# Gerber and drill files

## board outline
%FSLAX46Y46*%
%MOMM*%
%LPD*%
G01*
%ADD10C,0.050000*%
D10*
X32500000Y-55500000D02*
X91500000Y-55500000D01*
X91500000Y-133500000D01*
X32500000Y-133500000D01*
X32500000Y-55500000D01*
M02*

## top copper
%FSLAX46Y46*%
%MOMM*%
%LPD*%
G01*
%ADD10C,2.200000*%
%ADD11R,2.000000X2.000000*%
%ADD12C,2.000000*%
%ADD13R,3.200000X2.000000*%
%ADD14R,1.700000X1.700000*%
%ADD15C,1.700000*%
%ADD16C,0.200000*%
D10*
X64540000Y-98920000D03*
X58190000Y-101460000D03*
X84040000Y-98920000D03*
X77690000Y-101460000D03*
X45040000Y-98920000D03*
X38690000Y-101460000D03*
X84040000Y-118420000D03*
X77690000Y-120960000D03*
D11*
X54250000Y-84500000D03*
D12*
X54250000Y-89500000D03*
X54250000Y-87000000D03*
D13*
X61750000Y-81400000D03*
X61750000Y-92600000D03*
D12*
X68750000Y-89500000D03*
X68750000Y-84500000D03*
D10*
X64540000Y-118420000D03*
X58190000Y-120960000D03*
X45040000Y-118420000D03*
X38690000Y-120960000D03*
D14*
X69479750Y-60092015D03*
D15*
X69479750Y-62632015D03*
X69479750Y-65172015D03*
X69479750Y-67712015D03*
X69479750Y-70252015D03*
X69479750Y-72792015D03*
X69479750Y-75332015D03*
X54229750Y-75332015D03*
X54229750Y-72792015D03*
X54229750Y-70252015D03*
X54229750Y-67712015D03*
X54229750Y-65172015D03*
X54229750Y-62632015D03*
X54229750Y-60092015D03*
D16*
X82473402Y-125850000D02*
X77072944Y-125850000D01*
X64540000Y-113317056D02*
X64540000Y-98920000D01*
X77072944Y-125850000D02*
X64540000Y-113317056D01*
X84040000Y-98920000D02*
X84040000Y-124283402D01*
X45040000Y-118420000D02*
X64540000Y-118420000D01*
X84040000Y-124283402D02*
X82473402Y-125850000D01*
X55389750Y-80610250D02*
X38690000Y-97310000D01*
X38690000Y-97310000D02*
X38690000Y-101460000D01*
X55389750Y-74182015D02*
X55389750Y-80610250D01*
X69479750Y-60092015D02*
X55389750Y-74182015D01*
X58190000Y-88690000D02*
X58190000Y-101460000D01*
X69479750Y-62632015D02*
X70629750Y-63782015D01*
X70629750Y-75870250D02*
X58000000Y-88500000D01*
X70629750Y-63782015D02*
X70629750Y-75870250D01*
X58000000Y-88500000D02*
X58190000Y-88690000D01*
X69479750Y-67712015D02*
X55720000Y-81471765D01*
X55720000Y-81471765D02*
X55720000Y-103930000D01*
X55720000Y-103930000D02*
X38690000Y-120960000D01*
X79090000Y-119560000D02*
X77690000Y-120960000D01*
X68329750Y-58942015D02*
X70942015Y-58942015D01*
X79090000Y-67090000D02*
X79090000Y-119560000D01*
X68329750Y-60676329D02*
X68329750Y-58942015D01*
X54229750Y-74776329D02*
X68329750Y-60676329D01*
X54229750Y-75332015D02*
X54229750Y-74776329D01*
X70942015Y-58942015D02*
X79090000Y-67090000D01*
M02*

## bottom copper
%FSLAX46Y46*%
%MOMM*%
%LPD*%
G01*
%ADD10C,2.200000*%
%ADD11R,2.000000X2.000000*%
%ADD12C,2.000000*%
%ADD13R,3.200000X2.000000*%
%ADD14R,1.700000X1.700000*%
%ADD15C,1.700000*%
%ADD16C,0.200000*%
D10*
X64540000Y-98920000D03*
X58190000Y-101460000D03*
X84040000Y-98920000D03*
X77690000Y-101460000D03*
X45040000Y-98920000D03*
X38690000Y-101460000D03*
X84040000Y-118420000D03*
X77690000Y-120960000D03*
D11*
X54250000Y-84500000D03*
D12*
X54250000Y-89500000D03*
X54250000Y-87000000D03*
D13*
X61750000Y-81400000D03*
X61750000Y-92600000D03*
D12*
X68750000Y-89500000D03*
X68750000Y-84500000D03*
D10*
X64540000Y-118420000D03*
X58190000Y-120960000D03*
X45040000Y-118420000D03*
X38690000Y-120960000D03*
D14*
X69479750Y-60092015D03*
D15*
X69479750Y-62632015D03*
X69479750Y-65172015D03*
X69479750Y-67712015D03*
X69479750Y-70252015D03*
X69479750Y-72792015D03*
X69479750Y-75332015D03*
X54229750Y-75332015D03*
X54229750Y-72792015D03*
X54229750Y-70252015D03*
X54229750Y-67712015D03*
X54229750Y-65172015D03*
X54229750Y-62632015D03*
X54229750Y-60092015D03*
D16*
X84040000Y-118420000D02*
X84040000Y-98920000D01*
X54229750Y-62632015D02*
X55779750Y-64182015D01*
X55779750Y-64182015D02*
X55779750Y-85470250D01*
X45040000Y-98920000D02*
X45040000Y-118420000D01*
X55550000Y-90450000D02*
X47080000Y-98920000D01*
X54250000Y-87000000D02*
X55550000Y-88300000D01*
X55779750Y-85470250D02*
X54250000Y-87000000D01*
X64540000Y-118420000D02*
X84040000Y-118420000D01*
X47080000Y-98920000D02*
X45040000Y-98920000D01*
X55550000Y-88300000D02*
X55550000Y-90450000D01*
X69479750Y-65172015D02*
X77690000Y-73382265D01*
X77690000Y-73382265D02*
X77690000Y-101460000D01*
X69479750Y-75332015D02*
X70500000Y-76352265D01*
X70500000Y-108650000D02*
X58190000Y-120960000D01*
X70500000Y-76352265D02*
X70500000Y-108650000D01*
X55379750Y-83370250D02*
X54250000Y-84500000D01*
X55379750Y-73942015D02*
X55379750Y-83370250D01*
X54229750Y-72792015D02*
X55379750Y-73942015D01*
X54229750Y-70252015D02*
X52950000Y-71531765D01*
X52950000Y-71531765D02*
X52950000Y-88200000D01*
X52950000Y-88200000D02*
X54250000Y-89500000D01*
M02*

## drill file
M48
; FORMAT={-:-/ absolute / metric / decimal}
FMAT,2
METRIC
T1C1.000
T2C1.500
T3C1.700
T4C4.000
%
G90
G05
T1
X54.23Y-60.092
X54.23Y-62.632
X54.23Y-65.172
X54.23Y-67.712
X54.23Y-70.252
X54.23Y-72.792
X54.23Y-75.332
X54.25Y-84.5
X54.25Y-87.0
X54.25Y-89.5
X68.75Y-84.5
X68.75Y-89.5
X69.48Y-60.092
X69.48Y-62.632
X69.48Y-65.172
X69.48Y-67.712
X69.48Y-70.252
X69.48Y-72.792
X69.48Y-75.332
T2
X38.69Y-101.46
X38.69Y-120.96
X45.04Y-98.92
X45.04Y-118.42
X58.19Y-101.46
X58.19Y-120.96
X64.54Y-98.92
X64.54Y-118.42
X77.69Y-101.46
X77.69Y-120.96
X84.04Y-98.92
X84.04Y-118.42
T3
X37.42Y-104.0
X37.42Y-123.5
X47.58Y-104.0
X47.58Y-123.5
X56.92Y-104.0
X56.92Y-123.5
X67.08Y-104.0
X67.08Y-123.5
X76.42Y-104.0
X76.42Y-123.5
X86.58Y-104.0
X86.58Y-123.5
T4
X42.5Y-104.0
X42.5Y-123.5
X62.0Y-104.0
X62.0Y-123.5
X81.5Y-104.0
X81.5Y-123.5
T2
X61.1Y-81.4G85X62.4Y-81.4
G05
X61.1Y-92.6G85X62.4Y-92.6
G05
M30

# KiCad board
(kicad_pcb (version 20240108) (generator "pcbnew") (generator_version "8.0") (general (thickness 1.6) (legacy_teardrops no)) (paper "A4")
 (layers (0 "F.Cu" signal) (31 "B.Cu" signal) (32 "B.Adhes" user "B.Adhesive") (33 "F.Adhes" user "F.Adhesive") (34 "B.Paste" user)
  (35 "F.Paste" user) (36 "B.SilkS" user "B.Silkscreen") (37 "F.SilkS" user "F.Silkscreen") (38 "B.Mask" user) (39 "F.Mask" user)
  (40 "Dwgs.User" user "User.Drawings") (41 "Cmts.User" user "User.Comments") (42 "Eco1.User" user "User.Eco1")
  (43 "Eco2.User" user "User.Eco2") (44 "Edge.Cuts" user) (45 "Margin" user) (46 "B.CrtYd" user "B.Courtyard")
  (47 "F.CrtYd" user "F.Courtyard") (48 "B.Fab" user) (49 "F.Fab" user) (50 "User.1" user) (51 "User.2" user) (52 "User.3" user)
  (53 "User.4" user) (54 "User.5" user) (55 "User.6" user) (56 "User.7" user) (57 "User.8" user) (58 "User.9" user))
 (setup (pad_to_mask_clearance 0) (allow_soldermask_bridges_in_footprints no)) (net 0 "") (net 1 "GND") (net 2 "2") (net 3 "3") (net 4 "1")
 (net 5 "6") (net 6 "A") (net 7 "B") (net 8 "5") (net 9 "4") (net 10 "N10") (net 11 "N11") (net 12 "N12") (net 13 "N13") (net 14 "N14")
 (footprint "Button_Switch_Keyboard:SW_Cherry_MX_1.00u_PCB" (layer "F.Cu") (at 64.54 98.92)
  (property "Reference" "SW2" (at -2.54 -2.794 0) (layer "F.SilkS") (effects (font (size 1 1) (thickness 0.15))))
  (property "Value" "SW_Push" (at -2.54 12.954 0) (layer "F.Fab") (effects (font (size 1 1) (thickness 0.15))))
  (pad "" np_thru_hole circle (at -7.62 5.08) (size 1.7 1.7) (drill 1.7) (layers "*.Cu" "*.Mask"))
  (pad "" np_thru_hole circle (at -2.54 5.08) (size 4 4) (drill 4) (layers "*.Cu" "*.Mask"))
  (pad "" np_thru_hole circle (at 2.54 5.08) (size 1.7 1.7) (drill 1.7) (layers "*.Cu" "*.Mask"))
  (pad "1" thru_hole circle (at 0 0) (size 2.2 2.2) (drill 1.5) (layers "*.Cu" "*.Mask") (remove_unused_layers no) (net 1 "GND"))
  (pad "2" thru_hole circle (at -6.35 2.54) (size 2.2 2.2) (drill 1.5) (layers "*.Cu" "*.Mask") (remove_unused_layers no) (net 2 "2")))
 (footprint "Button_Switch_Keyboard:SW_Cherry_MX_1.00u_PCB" (layer "F.Cu") (at 84.04 98.92)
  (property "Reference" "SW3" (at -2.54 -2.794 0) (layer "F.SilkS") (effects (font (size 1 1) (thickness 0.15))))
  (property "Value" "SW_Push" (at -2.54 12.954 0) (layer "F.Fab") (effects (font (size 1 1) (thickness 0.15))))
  (pad "" np_thru_hole circle (at -7.62 5.08) (size 1.7 1.7) (drill 1.7) (layers "*.Cu" "*.Mask"))
  (pad "" np_thru_hole circle (at -2.54 5.08) (size 4 4) (drill 4) (layers "*.Cu" "*.Mask"))
  (pad "" np_thru_hole circle (at 2.54 5.08) (size 1.7 1.7) (drill 1.7) (layers "*.Cu" "*.Mask"))
  (pad "1" thru_hole circle (at 0 0) (size 2.2 2.2) (drill 1.5) (layers "*.Cu" "*.Mask") (remove_unused_layers no) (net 1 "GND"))
  (pad "2" thru_hole circle (at -6.35 2.54) (size 2.2 2.2) (drill 1.5) (layers "*.Cu" "*.Mask") (remove_unused_layers no) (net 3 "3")))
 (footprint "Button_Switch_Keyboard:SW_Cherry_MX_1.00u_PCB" (layer "F.Cu") (at 45.04 98.92)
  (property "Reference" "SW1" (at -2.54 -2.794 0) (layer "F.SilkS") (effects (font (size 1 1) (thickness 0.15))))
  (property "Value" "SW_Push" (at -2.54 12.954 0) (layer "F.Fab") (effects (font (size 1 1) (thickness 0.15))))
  (pad "" np_thru_hole circle (at -7.62 5.08) (size 1.7 1.7) (drill 1.7) (layers "*.Cu" "*.Mask"))
  (pad "" np_thru_hole circle (at -2.54 5.08) (size 4 4) (drill 4) (layers "*.Cu" "*.Mask"))
  (pad "" np_thru_hole circle (at 2.54 5.08) (size 1.7 1.7) (drill 1.7) (layers "*.Cu" "*.Mask"))
  (pad "1" thru_hole circle (at 0 0) (size 2.2 2.2) (drill 1.5) (layers "*.Cu" "*.Mask") (remove_unused_layers no) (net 1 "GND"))
  (pad "2" thru_hole circle (at -6.35 2.54) (size 2.2 2.2) (drill 1.5) (layers "*.Cu" "*.Mask") (remove_unused_layers no) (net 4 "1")))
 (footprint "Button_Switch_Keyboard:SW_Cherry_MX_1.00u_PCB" (layer "F.Cu") (at 84.04 118.42)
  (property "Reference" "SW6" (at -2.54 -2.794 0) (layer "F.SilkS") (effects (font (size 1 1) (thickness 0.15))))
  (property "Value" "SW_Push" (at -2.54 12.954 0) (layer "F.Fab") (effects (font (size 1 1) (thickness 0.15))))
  (pad "" np_thru_hole circle (at -7.62 5.08) (size 1.7 1.7) (drill 1.7) (layers "*.Cu" "*.Mask"))
  (pad "" np_thru_hole circle (at -2.54 5.08) (size 4 4) (drill 4) (layers "*.Cu" "*.Mask"))
  (pad "" np_thru_hole circle (at 2.54 5.08) (size 1.7 1.7) (drill 1.7) (layers "*.Cu" "*.Mask"))
  (pad "1" thru_hole circle (at 0 0) (size 2.2 2.2) (drill 1.5) (layers "*.Cu" "*.Mask") (remove_unused_layers no) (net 1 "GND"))
  (pad "2" thru_hole circle (at -6.35 2.54) (size 2.2 2.2) (drill 1.5) (layers "*.Cu" "*.Mask") (remove_unused_layers no) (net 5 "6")))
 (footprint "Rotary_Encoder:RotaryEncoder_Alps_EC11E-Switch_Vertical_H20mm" (layer "F.Cu") (at 54.25 84.5)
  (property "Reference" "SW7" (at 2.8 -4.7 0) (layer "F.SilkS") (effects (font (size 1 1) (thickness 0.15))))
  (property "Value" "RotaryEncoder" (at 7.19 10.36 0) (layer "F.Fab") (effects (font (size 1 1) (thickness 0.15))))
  (pad "A" thru_hole rect (at 0 0) (size 2 2) (drill 1) (layers "*.Cu" "*.Mask") (remove_unused_layers no) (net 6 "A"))
  (pad "B" thru_hole circle (at 0 5) (size 2 2) (drill 1) (layers "*.Cu" "*.Mask") (remove_unused_layers no) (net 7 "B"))
  (pad "C" thru_hole circle (at 0 2.5) (size 2 2) (drill 1) (layers "*.Cu" "*.Mask") (remove_unused_layers no) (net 1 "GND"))
  (pad "MP" thru_hole rect (at 7.5 -3.1) (size 3.2 2) (drill oval 2.8 1.5) (layers "*.Cu" "*.Mask") (remove_unused_layers no))
  (pad "MP" thru_hole rect (at 7.5 8.1) (size 3.2 2) (drill oval 2.8 1.5) (layers "*.Cu" "*.Mask") (remove_unused_layers no))
  (pad "S1" thru_hole circle (at 14.5 5) (size 2 2) (drill 1) (layers "*.Cu" "*.Mask") (remove_unused_layers no))
  (pad "S2" thru_hole circle (at 14.5 0) (size 2 2) (drill 1) (layers "*.Cu" "*.Mask") (remove_unused_layers no)))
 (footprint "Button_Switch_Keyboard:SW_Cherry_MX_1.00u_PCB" (layer "F.Cu") (at 64.54 118.42)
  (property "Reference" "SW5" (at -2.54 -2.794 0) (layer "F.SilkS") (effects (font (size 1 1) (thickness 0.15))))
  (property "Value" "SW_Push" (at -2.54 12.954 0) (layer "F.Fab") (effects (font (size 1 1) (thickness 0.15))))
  (pad "" np_thru_hole circle (at -7.62 5.08) (size 1.7 1.7) (drill 1.7) (layers "*.Cu" "*.Mask"))
  (pad "" np_thru_hole circle (at -2.54 5.08) (size 4 4) (drill 4) (layers "*.Cu" "*.Mask"))
  (pad "" np_thru_hole circle (at 2.54 5.08) (size 1.7 1.7) (drill 1.7) (layers "*.Cu" "*.Mask"))
  (pad "1" thru_hole circle (at 0 0) (size 2.2 2.2) (drill 1.5) (layers "*.Cu" "*.Mask") (remove_unused_layers no) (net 1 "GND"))
  (pad "2" thru_hole circle (at -6.35 2.54) (size 2.2 2.2) (drill 1.5) (layers "*.Cu" "*.Mask") (remove_unused_layers no) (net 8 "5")))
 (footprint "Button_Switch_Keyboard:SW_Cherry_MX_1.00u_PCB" (layer "F.Cu") (at 45.04 118.42)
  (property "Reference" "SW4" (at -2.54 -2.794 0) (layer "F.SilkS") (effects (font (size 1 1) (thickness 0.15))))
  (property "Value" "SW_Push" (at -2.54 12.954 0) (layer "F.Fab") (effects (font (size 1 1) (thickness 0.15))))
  (pad "" np_thru_hole circle (at -7.62 5.08) (size 1.7 1.7) (drill 1.7) (layers "*.Cu" "*.Mask"))
  (pad "" np_thru_hole circle (at -2.54 5.08) (size 4 4) (drill 4) (layers "*.Cu" "*.Mask"))
  (pad "" np_thru_hole circle (at 2.54 5.08) (size 1.7 1.7) (drill 1.7) (layers "*.Cu" "*.Mask"))
  (pad "1" thru_hole circle (at 0 0) (size 2.2 2.2) (drill 1.5) (layers "*.Cu" "*.Mask") (remove_unused_layers no) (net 1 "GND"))
  (pad "2" thru_hole circle (at -6.35 2.54) (size 2.2 2.2) (drill 1.5) (layers "*.Cu" "*.Mask") (remove_unused_layers no) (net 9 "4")))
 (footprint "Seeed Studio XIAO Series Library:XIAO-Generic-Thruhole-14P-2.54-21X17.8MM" (layer "B.Cu") (at 61.85475 67.712015 180)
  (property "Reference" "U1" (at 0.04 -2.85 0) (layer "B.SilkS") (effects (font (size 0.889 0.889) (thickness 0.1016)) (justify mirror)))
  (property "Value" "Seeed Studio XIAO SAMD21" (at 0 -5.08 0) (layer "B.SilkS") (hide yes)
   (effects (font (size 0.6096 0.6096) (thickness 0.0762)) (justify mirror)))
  (pad "1" thru_hole rect (at -7.625 7.62 180) (size 1.7 1.7) (drill 1) (layers "*.Cu" "*.Mask") (remove_unused_layers no) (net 4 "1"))
  (pad "2" thru_hole circle (at -7.625 5.08 180) (size 1.7 1.7) (drill 1) (layers "*.Cu" "*.Mask") (remove_unused_layers no) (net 2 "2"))
  (pad "3" thru_hole circle (at -7.625 2.54 180) (size 1.7 1.7) (drill 1) (layers "*.Cu" "*.Mask") (remove_unused_layers no) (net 3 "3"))
  (pad "4" thru_hole circle (at -7.625 0 180) (size 1.7 1.7) (drill 1) (layers "*.Cu" "*.Mask") (remove_unused_layers no) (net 9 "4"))
  (pad "5" thru_hole circle (at -7.625 -2.54 180) (size 1.7 1.7) (drill 1) (layers "*.Cu" "*.Mask") (remove_unused_layers no) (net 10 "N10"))
  (pad "6" thru_hole circle (at -7.625 -5.08) (size 1.7 1.7) (drill 1) (layers "*.Cu" "*.Mask") (remove_unused_layers no) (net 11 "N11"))
  (pad "7" thru_hole circle (at -7.625 -7.62 180) (size 1.7 1.7) (drill 1) (layers "*.Cu" "*.Mask") (remove_unused_layers no) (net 8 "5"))
  (pad "8" thru_hole circle (at 7.625 -7.62 180) (size 1.7 1.7) (drill 1) (layers "*.Cu" "*.Mask") (remove_unused_layers no) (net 5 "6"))
  (pad "9" thru_hole circle (at 7.625 -5.08 180) (size 1.7 1.7) (drill 1) (layers "*.Cu" "*.Mask") (remove_unused_layers no) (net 6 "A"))
  (pad "10" thru_hole circle (at 7.625 -2.54 180) (size 1.7 1.7) (drill 1) (layers "*.Cu" "*.Mask") (remove_unused_layers no) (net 7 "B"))
  (pad "11" thru_hole circle (at 7.625 0 180) (size 1.7 1.7) (drill 1) (layers "*.Cu" "*.Mask") (remove_unused_layers no) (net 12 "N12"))
  (pad "12" thru_hole circle (at 7.625 2.54 180) (size 1.7 1.7) (drill 1) (layers "*.Cu" "*.Mask") (remove_unused_layers no) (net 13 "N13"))
  (pad "13" thru_hole circle (at 7.625 5.08 180) (size 1.7 1.7) (drill 1) (layers "*.Cu" "*.Mask") (remove_unused_layers no) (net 1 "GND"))
  (pad "14" thru_hole circle (at 7.625 7.62 180) (size 1.7 1.7) (drill 1) (layers "*.Cu" "*.Mask") (remove_unused_layers no) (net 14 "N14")))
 (gr_rect (start 32.5 55.5) (end 91.5 133.5) (stroke (width 0.05) (type default)) (fill none) (layer "Edge.Cuts"))
 (segment (start 82.473402 125.85) (end 77.072944 125.85) (width 0.2) (layer "F.Cu") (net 1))
 (segment (start 64.54 113.317056) (end 64.54 98.92) (width 0.2) (layer "F.Cu") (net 1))
 (segment (start 77.072944 125.85) (end 64.54 113.317056) (width 0.2) (layer "F.Cu") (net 1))
 (segment (start 84.04 98.92) (end 84.04 124.283402) (width 0.2) (layer "F.Cu") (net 1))
 (segment (start 45.04 118.42) (end 64.54 118.42) (width 0.2) (layer "F.Cu") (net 1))
 (segment (start 84.04 124.283402) (end 82.473402 125.85) (width 0.2) (layer "F.Cu") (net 1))
 (segment (start 84.04 118.42) (end 84.04 98.92) (width 0.2) (layer "B.Cu") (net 1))
 (segment (start 54.22975 62.632015) (end 55.77975 64.182015) (width 0.2) (layer "B.Cu") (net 1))
 (segment (start 55.77975 64.182015) (end 55.77975 85.47025) (width 0.2) (layer "B.Cu") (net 1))
 (segment (start 45.04 98.92) (end 45.04 118.42) (width 0.2) (layer "B.Cu") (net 1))
 (segment (start 55.55 90.45) (end 47.08 98.92) (width 0.2) (layer "B.Cu") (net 1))
 (segment (start 54.25 87) (end 55.55 88.3) (width 0.2) (layer "B.Cu") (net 1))
 (segment (start 55.77975 85.47025) (end 54.25 87) (width 0.2) (layer "B.Cu") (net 1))
 (segment (start 64.54 118.42) (end 84.04 118.42) (width 0.2) (layer "B.Cu") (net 1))
 (segment (start 47.08 98.92) (end 45.04 98.92) (width 0.2) (layer "B.Cu") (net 1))
 (segment (start 55.55 88.3) (end 55.55 90.45) (width 0.2) (layer "B.Cu") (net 1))
 (segment (start 55.38975 80.61025) (end 38.69 97.31) (width 0.2) (layer "F.Cu") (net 4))
 (segment (start 38.69 97.31) (end 38.69 101.46) (width 0.2) (layer "F.Cu") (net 4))
 (segment (start 55.38975 74.182015) (end 55.38975 80.61025) (width 0.2) (layer "F.Cu") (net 4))
 (segment (start 69.47975 60.092015) (end 55.38975 74.182015) (width 0.2) (layer "F.Cu") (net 4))
 (segment (start 58.19 88.69) (end 58.19 101.46) (width 0.2) (layer "F.Cu") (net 2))
 (segment (start 69.47975 62.632015) (end 70.62975 63.782015) (width 0.2) (layer "F.Cu") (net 2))
 (segment (start 70.62975 75.87025) (end 58 88.5) (width 0.2) (layer "F.Cu") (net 2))
 (segment (start 70.62975 63.782015) (end 70.62975 75.87025) (width 0.2) (layer "F.Cu") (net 2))
 (segment (start 58 88.5) (end 58.19 88.69) (width 0.2) (layer "F.Cu") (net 2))
 (segment (start 69.47975 65.172015) (end 77.69 73.382265) (width 0.2) (layer "B.Cu") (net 3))
 (segment (start 77.69 73.382265) (end 77.69 101.46) (width 0.2) (layer "B.Cu") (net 3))
 (segment (start 69.47975 67.712015) (end 55.72 81.471765) (width 0.2) (layer "F.Cu") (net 9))
 (segment (start 55.72 81.471765) (end 55.72 103.93) (width 0.2) (layer "F.Cu") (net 9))
 (segment (start 55.72 103.93) (end 38.69 120.96) (width 0.2) (layer "F.Cu") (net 9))
 (segment (start 69.47975 75.332015) (end 70.5 76.352265) (width 0.2) (layer "B.Cu") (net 8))
 (segment (start 70.5 108.65) (end 58.19 120.96) (width 0.2) (layer "B.Cu") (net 8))
 (segment (start 70.5 76.352265) (end 70.5 108.65) (width 0.2) (layer "B.Cu") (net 8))
 (segment (start 79.09 119.56) (end 77.69 120.96) (width 0.2) (layer "F.Cu") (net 5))
 (segment (start 68.32975 58.942015) (end 70.942015 58.942015) (width 0.2) (layer "F.Cu") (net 5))
 (segment (start 79.09 67.09) (end 79.09 119.56) (width 0.2) (layer "F.Cu") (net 5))
 (segment (start 68.32975 60.676329) (end 68.32975 58.942015) (width 0.2) (layer "F.Cu") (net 5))
 (segment (start 54.22975 74.776329) (end 68.32975 60.676329) (width 0.2) (layer "F.Cu") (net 5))
 (segment (start 54.22975 75.332015) (end 54.22975 74.776329) (width 0.2) (layer "F.Cu") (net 5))
 (segment (start 70.942015 58.942015) (end 79.09 67.09) (width 0.2) (layer "F.Cu") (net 5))
 (segment (start 55.37975 83.37025) (end 54.25 84.5) (width 0.2) (layer "B.Cu") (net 6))
 (segment (start 55.37975 73.942015) (end 55.37975 83.37025) (width 0.2) (layer "B.Cu") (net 6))
 (segment (start 54.22975 72.792015) (end 55.37975 73.942015) (width 0.2) (layer "B.Cu") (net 6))
 (segment (start 54.22975 70.252015) (end 52.95 71.531765) (width 0.2) (layer "B.Cu") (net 7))
 (segment (start 52.95 71.531765) (end 52.95 88.2) (width 0.2) (layer "B.Cu") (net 7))
 (segment (start 52.95 88.2) (end 54.25 89.5) (width 0.2) (layer "B.Cu") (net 7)))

